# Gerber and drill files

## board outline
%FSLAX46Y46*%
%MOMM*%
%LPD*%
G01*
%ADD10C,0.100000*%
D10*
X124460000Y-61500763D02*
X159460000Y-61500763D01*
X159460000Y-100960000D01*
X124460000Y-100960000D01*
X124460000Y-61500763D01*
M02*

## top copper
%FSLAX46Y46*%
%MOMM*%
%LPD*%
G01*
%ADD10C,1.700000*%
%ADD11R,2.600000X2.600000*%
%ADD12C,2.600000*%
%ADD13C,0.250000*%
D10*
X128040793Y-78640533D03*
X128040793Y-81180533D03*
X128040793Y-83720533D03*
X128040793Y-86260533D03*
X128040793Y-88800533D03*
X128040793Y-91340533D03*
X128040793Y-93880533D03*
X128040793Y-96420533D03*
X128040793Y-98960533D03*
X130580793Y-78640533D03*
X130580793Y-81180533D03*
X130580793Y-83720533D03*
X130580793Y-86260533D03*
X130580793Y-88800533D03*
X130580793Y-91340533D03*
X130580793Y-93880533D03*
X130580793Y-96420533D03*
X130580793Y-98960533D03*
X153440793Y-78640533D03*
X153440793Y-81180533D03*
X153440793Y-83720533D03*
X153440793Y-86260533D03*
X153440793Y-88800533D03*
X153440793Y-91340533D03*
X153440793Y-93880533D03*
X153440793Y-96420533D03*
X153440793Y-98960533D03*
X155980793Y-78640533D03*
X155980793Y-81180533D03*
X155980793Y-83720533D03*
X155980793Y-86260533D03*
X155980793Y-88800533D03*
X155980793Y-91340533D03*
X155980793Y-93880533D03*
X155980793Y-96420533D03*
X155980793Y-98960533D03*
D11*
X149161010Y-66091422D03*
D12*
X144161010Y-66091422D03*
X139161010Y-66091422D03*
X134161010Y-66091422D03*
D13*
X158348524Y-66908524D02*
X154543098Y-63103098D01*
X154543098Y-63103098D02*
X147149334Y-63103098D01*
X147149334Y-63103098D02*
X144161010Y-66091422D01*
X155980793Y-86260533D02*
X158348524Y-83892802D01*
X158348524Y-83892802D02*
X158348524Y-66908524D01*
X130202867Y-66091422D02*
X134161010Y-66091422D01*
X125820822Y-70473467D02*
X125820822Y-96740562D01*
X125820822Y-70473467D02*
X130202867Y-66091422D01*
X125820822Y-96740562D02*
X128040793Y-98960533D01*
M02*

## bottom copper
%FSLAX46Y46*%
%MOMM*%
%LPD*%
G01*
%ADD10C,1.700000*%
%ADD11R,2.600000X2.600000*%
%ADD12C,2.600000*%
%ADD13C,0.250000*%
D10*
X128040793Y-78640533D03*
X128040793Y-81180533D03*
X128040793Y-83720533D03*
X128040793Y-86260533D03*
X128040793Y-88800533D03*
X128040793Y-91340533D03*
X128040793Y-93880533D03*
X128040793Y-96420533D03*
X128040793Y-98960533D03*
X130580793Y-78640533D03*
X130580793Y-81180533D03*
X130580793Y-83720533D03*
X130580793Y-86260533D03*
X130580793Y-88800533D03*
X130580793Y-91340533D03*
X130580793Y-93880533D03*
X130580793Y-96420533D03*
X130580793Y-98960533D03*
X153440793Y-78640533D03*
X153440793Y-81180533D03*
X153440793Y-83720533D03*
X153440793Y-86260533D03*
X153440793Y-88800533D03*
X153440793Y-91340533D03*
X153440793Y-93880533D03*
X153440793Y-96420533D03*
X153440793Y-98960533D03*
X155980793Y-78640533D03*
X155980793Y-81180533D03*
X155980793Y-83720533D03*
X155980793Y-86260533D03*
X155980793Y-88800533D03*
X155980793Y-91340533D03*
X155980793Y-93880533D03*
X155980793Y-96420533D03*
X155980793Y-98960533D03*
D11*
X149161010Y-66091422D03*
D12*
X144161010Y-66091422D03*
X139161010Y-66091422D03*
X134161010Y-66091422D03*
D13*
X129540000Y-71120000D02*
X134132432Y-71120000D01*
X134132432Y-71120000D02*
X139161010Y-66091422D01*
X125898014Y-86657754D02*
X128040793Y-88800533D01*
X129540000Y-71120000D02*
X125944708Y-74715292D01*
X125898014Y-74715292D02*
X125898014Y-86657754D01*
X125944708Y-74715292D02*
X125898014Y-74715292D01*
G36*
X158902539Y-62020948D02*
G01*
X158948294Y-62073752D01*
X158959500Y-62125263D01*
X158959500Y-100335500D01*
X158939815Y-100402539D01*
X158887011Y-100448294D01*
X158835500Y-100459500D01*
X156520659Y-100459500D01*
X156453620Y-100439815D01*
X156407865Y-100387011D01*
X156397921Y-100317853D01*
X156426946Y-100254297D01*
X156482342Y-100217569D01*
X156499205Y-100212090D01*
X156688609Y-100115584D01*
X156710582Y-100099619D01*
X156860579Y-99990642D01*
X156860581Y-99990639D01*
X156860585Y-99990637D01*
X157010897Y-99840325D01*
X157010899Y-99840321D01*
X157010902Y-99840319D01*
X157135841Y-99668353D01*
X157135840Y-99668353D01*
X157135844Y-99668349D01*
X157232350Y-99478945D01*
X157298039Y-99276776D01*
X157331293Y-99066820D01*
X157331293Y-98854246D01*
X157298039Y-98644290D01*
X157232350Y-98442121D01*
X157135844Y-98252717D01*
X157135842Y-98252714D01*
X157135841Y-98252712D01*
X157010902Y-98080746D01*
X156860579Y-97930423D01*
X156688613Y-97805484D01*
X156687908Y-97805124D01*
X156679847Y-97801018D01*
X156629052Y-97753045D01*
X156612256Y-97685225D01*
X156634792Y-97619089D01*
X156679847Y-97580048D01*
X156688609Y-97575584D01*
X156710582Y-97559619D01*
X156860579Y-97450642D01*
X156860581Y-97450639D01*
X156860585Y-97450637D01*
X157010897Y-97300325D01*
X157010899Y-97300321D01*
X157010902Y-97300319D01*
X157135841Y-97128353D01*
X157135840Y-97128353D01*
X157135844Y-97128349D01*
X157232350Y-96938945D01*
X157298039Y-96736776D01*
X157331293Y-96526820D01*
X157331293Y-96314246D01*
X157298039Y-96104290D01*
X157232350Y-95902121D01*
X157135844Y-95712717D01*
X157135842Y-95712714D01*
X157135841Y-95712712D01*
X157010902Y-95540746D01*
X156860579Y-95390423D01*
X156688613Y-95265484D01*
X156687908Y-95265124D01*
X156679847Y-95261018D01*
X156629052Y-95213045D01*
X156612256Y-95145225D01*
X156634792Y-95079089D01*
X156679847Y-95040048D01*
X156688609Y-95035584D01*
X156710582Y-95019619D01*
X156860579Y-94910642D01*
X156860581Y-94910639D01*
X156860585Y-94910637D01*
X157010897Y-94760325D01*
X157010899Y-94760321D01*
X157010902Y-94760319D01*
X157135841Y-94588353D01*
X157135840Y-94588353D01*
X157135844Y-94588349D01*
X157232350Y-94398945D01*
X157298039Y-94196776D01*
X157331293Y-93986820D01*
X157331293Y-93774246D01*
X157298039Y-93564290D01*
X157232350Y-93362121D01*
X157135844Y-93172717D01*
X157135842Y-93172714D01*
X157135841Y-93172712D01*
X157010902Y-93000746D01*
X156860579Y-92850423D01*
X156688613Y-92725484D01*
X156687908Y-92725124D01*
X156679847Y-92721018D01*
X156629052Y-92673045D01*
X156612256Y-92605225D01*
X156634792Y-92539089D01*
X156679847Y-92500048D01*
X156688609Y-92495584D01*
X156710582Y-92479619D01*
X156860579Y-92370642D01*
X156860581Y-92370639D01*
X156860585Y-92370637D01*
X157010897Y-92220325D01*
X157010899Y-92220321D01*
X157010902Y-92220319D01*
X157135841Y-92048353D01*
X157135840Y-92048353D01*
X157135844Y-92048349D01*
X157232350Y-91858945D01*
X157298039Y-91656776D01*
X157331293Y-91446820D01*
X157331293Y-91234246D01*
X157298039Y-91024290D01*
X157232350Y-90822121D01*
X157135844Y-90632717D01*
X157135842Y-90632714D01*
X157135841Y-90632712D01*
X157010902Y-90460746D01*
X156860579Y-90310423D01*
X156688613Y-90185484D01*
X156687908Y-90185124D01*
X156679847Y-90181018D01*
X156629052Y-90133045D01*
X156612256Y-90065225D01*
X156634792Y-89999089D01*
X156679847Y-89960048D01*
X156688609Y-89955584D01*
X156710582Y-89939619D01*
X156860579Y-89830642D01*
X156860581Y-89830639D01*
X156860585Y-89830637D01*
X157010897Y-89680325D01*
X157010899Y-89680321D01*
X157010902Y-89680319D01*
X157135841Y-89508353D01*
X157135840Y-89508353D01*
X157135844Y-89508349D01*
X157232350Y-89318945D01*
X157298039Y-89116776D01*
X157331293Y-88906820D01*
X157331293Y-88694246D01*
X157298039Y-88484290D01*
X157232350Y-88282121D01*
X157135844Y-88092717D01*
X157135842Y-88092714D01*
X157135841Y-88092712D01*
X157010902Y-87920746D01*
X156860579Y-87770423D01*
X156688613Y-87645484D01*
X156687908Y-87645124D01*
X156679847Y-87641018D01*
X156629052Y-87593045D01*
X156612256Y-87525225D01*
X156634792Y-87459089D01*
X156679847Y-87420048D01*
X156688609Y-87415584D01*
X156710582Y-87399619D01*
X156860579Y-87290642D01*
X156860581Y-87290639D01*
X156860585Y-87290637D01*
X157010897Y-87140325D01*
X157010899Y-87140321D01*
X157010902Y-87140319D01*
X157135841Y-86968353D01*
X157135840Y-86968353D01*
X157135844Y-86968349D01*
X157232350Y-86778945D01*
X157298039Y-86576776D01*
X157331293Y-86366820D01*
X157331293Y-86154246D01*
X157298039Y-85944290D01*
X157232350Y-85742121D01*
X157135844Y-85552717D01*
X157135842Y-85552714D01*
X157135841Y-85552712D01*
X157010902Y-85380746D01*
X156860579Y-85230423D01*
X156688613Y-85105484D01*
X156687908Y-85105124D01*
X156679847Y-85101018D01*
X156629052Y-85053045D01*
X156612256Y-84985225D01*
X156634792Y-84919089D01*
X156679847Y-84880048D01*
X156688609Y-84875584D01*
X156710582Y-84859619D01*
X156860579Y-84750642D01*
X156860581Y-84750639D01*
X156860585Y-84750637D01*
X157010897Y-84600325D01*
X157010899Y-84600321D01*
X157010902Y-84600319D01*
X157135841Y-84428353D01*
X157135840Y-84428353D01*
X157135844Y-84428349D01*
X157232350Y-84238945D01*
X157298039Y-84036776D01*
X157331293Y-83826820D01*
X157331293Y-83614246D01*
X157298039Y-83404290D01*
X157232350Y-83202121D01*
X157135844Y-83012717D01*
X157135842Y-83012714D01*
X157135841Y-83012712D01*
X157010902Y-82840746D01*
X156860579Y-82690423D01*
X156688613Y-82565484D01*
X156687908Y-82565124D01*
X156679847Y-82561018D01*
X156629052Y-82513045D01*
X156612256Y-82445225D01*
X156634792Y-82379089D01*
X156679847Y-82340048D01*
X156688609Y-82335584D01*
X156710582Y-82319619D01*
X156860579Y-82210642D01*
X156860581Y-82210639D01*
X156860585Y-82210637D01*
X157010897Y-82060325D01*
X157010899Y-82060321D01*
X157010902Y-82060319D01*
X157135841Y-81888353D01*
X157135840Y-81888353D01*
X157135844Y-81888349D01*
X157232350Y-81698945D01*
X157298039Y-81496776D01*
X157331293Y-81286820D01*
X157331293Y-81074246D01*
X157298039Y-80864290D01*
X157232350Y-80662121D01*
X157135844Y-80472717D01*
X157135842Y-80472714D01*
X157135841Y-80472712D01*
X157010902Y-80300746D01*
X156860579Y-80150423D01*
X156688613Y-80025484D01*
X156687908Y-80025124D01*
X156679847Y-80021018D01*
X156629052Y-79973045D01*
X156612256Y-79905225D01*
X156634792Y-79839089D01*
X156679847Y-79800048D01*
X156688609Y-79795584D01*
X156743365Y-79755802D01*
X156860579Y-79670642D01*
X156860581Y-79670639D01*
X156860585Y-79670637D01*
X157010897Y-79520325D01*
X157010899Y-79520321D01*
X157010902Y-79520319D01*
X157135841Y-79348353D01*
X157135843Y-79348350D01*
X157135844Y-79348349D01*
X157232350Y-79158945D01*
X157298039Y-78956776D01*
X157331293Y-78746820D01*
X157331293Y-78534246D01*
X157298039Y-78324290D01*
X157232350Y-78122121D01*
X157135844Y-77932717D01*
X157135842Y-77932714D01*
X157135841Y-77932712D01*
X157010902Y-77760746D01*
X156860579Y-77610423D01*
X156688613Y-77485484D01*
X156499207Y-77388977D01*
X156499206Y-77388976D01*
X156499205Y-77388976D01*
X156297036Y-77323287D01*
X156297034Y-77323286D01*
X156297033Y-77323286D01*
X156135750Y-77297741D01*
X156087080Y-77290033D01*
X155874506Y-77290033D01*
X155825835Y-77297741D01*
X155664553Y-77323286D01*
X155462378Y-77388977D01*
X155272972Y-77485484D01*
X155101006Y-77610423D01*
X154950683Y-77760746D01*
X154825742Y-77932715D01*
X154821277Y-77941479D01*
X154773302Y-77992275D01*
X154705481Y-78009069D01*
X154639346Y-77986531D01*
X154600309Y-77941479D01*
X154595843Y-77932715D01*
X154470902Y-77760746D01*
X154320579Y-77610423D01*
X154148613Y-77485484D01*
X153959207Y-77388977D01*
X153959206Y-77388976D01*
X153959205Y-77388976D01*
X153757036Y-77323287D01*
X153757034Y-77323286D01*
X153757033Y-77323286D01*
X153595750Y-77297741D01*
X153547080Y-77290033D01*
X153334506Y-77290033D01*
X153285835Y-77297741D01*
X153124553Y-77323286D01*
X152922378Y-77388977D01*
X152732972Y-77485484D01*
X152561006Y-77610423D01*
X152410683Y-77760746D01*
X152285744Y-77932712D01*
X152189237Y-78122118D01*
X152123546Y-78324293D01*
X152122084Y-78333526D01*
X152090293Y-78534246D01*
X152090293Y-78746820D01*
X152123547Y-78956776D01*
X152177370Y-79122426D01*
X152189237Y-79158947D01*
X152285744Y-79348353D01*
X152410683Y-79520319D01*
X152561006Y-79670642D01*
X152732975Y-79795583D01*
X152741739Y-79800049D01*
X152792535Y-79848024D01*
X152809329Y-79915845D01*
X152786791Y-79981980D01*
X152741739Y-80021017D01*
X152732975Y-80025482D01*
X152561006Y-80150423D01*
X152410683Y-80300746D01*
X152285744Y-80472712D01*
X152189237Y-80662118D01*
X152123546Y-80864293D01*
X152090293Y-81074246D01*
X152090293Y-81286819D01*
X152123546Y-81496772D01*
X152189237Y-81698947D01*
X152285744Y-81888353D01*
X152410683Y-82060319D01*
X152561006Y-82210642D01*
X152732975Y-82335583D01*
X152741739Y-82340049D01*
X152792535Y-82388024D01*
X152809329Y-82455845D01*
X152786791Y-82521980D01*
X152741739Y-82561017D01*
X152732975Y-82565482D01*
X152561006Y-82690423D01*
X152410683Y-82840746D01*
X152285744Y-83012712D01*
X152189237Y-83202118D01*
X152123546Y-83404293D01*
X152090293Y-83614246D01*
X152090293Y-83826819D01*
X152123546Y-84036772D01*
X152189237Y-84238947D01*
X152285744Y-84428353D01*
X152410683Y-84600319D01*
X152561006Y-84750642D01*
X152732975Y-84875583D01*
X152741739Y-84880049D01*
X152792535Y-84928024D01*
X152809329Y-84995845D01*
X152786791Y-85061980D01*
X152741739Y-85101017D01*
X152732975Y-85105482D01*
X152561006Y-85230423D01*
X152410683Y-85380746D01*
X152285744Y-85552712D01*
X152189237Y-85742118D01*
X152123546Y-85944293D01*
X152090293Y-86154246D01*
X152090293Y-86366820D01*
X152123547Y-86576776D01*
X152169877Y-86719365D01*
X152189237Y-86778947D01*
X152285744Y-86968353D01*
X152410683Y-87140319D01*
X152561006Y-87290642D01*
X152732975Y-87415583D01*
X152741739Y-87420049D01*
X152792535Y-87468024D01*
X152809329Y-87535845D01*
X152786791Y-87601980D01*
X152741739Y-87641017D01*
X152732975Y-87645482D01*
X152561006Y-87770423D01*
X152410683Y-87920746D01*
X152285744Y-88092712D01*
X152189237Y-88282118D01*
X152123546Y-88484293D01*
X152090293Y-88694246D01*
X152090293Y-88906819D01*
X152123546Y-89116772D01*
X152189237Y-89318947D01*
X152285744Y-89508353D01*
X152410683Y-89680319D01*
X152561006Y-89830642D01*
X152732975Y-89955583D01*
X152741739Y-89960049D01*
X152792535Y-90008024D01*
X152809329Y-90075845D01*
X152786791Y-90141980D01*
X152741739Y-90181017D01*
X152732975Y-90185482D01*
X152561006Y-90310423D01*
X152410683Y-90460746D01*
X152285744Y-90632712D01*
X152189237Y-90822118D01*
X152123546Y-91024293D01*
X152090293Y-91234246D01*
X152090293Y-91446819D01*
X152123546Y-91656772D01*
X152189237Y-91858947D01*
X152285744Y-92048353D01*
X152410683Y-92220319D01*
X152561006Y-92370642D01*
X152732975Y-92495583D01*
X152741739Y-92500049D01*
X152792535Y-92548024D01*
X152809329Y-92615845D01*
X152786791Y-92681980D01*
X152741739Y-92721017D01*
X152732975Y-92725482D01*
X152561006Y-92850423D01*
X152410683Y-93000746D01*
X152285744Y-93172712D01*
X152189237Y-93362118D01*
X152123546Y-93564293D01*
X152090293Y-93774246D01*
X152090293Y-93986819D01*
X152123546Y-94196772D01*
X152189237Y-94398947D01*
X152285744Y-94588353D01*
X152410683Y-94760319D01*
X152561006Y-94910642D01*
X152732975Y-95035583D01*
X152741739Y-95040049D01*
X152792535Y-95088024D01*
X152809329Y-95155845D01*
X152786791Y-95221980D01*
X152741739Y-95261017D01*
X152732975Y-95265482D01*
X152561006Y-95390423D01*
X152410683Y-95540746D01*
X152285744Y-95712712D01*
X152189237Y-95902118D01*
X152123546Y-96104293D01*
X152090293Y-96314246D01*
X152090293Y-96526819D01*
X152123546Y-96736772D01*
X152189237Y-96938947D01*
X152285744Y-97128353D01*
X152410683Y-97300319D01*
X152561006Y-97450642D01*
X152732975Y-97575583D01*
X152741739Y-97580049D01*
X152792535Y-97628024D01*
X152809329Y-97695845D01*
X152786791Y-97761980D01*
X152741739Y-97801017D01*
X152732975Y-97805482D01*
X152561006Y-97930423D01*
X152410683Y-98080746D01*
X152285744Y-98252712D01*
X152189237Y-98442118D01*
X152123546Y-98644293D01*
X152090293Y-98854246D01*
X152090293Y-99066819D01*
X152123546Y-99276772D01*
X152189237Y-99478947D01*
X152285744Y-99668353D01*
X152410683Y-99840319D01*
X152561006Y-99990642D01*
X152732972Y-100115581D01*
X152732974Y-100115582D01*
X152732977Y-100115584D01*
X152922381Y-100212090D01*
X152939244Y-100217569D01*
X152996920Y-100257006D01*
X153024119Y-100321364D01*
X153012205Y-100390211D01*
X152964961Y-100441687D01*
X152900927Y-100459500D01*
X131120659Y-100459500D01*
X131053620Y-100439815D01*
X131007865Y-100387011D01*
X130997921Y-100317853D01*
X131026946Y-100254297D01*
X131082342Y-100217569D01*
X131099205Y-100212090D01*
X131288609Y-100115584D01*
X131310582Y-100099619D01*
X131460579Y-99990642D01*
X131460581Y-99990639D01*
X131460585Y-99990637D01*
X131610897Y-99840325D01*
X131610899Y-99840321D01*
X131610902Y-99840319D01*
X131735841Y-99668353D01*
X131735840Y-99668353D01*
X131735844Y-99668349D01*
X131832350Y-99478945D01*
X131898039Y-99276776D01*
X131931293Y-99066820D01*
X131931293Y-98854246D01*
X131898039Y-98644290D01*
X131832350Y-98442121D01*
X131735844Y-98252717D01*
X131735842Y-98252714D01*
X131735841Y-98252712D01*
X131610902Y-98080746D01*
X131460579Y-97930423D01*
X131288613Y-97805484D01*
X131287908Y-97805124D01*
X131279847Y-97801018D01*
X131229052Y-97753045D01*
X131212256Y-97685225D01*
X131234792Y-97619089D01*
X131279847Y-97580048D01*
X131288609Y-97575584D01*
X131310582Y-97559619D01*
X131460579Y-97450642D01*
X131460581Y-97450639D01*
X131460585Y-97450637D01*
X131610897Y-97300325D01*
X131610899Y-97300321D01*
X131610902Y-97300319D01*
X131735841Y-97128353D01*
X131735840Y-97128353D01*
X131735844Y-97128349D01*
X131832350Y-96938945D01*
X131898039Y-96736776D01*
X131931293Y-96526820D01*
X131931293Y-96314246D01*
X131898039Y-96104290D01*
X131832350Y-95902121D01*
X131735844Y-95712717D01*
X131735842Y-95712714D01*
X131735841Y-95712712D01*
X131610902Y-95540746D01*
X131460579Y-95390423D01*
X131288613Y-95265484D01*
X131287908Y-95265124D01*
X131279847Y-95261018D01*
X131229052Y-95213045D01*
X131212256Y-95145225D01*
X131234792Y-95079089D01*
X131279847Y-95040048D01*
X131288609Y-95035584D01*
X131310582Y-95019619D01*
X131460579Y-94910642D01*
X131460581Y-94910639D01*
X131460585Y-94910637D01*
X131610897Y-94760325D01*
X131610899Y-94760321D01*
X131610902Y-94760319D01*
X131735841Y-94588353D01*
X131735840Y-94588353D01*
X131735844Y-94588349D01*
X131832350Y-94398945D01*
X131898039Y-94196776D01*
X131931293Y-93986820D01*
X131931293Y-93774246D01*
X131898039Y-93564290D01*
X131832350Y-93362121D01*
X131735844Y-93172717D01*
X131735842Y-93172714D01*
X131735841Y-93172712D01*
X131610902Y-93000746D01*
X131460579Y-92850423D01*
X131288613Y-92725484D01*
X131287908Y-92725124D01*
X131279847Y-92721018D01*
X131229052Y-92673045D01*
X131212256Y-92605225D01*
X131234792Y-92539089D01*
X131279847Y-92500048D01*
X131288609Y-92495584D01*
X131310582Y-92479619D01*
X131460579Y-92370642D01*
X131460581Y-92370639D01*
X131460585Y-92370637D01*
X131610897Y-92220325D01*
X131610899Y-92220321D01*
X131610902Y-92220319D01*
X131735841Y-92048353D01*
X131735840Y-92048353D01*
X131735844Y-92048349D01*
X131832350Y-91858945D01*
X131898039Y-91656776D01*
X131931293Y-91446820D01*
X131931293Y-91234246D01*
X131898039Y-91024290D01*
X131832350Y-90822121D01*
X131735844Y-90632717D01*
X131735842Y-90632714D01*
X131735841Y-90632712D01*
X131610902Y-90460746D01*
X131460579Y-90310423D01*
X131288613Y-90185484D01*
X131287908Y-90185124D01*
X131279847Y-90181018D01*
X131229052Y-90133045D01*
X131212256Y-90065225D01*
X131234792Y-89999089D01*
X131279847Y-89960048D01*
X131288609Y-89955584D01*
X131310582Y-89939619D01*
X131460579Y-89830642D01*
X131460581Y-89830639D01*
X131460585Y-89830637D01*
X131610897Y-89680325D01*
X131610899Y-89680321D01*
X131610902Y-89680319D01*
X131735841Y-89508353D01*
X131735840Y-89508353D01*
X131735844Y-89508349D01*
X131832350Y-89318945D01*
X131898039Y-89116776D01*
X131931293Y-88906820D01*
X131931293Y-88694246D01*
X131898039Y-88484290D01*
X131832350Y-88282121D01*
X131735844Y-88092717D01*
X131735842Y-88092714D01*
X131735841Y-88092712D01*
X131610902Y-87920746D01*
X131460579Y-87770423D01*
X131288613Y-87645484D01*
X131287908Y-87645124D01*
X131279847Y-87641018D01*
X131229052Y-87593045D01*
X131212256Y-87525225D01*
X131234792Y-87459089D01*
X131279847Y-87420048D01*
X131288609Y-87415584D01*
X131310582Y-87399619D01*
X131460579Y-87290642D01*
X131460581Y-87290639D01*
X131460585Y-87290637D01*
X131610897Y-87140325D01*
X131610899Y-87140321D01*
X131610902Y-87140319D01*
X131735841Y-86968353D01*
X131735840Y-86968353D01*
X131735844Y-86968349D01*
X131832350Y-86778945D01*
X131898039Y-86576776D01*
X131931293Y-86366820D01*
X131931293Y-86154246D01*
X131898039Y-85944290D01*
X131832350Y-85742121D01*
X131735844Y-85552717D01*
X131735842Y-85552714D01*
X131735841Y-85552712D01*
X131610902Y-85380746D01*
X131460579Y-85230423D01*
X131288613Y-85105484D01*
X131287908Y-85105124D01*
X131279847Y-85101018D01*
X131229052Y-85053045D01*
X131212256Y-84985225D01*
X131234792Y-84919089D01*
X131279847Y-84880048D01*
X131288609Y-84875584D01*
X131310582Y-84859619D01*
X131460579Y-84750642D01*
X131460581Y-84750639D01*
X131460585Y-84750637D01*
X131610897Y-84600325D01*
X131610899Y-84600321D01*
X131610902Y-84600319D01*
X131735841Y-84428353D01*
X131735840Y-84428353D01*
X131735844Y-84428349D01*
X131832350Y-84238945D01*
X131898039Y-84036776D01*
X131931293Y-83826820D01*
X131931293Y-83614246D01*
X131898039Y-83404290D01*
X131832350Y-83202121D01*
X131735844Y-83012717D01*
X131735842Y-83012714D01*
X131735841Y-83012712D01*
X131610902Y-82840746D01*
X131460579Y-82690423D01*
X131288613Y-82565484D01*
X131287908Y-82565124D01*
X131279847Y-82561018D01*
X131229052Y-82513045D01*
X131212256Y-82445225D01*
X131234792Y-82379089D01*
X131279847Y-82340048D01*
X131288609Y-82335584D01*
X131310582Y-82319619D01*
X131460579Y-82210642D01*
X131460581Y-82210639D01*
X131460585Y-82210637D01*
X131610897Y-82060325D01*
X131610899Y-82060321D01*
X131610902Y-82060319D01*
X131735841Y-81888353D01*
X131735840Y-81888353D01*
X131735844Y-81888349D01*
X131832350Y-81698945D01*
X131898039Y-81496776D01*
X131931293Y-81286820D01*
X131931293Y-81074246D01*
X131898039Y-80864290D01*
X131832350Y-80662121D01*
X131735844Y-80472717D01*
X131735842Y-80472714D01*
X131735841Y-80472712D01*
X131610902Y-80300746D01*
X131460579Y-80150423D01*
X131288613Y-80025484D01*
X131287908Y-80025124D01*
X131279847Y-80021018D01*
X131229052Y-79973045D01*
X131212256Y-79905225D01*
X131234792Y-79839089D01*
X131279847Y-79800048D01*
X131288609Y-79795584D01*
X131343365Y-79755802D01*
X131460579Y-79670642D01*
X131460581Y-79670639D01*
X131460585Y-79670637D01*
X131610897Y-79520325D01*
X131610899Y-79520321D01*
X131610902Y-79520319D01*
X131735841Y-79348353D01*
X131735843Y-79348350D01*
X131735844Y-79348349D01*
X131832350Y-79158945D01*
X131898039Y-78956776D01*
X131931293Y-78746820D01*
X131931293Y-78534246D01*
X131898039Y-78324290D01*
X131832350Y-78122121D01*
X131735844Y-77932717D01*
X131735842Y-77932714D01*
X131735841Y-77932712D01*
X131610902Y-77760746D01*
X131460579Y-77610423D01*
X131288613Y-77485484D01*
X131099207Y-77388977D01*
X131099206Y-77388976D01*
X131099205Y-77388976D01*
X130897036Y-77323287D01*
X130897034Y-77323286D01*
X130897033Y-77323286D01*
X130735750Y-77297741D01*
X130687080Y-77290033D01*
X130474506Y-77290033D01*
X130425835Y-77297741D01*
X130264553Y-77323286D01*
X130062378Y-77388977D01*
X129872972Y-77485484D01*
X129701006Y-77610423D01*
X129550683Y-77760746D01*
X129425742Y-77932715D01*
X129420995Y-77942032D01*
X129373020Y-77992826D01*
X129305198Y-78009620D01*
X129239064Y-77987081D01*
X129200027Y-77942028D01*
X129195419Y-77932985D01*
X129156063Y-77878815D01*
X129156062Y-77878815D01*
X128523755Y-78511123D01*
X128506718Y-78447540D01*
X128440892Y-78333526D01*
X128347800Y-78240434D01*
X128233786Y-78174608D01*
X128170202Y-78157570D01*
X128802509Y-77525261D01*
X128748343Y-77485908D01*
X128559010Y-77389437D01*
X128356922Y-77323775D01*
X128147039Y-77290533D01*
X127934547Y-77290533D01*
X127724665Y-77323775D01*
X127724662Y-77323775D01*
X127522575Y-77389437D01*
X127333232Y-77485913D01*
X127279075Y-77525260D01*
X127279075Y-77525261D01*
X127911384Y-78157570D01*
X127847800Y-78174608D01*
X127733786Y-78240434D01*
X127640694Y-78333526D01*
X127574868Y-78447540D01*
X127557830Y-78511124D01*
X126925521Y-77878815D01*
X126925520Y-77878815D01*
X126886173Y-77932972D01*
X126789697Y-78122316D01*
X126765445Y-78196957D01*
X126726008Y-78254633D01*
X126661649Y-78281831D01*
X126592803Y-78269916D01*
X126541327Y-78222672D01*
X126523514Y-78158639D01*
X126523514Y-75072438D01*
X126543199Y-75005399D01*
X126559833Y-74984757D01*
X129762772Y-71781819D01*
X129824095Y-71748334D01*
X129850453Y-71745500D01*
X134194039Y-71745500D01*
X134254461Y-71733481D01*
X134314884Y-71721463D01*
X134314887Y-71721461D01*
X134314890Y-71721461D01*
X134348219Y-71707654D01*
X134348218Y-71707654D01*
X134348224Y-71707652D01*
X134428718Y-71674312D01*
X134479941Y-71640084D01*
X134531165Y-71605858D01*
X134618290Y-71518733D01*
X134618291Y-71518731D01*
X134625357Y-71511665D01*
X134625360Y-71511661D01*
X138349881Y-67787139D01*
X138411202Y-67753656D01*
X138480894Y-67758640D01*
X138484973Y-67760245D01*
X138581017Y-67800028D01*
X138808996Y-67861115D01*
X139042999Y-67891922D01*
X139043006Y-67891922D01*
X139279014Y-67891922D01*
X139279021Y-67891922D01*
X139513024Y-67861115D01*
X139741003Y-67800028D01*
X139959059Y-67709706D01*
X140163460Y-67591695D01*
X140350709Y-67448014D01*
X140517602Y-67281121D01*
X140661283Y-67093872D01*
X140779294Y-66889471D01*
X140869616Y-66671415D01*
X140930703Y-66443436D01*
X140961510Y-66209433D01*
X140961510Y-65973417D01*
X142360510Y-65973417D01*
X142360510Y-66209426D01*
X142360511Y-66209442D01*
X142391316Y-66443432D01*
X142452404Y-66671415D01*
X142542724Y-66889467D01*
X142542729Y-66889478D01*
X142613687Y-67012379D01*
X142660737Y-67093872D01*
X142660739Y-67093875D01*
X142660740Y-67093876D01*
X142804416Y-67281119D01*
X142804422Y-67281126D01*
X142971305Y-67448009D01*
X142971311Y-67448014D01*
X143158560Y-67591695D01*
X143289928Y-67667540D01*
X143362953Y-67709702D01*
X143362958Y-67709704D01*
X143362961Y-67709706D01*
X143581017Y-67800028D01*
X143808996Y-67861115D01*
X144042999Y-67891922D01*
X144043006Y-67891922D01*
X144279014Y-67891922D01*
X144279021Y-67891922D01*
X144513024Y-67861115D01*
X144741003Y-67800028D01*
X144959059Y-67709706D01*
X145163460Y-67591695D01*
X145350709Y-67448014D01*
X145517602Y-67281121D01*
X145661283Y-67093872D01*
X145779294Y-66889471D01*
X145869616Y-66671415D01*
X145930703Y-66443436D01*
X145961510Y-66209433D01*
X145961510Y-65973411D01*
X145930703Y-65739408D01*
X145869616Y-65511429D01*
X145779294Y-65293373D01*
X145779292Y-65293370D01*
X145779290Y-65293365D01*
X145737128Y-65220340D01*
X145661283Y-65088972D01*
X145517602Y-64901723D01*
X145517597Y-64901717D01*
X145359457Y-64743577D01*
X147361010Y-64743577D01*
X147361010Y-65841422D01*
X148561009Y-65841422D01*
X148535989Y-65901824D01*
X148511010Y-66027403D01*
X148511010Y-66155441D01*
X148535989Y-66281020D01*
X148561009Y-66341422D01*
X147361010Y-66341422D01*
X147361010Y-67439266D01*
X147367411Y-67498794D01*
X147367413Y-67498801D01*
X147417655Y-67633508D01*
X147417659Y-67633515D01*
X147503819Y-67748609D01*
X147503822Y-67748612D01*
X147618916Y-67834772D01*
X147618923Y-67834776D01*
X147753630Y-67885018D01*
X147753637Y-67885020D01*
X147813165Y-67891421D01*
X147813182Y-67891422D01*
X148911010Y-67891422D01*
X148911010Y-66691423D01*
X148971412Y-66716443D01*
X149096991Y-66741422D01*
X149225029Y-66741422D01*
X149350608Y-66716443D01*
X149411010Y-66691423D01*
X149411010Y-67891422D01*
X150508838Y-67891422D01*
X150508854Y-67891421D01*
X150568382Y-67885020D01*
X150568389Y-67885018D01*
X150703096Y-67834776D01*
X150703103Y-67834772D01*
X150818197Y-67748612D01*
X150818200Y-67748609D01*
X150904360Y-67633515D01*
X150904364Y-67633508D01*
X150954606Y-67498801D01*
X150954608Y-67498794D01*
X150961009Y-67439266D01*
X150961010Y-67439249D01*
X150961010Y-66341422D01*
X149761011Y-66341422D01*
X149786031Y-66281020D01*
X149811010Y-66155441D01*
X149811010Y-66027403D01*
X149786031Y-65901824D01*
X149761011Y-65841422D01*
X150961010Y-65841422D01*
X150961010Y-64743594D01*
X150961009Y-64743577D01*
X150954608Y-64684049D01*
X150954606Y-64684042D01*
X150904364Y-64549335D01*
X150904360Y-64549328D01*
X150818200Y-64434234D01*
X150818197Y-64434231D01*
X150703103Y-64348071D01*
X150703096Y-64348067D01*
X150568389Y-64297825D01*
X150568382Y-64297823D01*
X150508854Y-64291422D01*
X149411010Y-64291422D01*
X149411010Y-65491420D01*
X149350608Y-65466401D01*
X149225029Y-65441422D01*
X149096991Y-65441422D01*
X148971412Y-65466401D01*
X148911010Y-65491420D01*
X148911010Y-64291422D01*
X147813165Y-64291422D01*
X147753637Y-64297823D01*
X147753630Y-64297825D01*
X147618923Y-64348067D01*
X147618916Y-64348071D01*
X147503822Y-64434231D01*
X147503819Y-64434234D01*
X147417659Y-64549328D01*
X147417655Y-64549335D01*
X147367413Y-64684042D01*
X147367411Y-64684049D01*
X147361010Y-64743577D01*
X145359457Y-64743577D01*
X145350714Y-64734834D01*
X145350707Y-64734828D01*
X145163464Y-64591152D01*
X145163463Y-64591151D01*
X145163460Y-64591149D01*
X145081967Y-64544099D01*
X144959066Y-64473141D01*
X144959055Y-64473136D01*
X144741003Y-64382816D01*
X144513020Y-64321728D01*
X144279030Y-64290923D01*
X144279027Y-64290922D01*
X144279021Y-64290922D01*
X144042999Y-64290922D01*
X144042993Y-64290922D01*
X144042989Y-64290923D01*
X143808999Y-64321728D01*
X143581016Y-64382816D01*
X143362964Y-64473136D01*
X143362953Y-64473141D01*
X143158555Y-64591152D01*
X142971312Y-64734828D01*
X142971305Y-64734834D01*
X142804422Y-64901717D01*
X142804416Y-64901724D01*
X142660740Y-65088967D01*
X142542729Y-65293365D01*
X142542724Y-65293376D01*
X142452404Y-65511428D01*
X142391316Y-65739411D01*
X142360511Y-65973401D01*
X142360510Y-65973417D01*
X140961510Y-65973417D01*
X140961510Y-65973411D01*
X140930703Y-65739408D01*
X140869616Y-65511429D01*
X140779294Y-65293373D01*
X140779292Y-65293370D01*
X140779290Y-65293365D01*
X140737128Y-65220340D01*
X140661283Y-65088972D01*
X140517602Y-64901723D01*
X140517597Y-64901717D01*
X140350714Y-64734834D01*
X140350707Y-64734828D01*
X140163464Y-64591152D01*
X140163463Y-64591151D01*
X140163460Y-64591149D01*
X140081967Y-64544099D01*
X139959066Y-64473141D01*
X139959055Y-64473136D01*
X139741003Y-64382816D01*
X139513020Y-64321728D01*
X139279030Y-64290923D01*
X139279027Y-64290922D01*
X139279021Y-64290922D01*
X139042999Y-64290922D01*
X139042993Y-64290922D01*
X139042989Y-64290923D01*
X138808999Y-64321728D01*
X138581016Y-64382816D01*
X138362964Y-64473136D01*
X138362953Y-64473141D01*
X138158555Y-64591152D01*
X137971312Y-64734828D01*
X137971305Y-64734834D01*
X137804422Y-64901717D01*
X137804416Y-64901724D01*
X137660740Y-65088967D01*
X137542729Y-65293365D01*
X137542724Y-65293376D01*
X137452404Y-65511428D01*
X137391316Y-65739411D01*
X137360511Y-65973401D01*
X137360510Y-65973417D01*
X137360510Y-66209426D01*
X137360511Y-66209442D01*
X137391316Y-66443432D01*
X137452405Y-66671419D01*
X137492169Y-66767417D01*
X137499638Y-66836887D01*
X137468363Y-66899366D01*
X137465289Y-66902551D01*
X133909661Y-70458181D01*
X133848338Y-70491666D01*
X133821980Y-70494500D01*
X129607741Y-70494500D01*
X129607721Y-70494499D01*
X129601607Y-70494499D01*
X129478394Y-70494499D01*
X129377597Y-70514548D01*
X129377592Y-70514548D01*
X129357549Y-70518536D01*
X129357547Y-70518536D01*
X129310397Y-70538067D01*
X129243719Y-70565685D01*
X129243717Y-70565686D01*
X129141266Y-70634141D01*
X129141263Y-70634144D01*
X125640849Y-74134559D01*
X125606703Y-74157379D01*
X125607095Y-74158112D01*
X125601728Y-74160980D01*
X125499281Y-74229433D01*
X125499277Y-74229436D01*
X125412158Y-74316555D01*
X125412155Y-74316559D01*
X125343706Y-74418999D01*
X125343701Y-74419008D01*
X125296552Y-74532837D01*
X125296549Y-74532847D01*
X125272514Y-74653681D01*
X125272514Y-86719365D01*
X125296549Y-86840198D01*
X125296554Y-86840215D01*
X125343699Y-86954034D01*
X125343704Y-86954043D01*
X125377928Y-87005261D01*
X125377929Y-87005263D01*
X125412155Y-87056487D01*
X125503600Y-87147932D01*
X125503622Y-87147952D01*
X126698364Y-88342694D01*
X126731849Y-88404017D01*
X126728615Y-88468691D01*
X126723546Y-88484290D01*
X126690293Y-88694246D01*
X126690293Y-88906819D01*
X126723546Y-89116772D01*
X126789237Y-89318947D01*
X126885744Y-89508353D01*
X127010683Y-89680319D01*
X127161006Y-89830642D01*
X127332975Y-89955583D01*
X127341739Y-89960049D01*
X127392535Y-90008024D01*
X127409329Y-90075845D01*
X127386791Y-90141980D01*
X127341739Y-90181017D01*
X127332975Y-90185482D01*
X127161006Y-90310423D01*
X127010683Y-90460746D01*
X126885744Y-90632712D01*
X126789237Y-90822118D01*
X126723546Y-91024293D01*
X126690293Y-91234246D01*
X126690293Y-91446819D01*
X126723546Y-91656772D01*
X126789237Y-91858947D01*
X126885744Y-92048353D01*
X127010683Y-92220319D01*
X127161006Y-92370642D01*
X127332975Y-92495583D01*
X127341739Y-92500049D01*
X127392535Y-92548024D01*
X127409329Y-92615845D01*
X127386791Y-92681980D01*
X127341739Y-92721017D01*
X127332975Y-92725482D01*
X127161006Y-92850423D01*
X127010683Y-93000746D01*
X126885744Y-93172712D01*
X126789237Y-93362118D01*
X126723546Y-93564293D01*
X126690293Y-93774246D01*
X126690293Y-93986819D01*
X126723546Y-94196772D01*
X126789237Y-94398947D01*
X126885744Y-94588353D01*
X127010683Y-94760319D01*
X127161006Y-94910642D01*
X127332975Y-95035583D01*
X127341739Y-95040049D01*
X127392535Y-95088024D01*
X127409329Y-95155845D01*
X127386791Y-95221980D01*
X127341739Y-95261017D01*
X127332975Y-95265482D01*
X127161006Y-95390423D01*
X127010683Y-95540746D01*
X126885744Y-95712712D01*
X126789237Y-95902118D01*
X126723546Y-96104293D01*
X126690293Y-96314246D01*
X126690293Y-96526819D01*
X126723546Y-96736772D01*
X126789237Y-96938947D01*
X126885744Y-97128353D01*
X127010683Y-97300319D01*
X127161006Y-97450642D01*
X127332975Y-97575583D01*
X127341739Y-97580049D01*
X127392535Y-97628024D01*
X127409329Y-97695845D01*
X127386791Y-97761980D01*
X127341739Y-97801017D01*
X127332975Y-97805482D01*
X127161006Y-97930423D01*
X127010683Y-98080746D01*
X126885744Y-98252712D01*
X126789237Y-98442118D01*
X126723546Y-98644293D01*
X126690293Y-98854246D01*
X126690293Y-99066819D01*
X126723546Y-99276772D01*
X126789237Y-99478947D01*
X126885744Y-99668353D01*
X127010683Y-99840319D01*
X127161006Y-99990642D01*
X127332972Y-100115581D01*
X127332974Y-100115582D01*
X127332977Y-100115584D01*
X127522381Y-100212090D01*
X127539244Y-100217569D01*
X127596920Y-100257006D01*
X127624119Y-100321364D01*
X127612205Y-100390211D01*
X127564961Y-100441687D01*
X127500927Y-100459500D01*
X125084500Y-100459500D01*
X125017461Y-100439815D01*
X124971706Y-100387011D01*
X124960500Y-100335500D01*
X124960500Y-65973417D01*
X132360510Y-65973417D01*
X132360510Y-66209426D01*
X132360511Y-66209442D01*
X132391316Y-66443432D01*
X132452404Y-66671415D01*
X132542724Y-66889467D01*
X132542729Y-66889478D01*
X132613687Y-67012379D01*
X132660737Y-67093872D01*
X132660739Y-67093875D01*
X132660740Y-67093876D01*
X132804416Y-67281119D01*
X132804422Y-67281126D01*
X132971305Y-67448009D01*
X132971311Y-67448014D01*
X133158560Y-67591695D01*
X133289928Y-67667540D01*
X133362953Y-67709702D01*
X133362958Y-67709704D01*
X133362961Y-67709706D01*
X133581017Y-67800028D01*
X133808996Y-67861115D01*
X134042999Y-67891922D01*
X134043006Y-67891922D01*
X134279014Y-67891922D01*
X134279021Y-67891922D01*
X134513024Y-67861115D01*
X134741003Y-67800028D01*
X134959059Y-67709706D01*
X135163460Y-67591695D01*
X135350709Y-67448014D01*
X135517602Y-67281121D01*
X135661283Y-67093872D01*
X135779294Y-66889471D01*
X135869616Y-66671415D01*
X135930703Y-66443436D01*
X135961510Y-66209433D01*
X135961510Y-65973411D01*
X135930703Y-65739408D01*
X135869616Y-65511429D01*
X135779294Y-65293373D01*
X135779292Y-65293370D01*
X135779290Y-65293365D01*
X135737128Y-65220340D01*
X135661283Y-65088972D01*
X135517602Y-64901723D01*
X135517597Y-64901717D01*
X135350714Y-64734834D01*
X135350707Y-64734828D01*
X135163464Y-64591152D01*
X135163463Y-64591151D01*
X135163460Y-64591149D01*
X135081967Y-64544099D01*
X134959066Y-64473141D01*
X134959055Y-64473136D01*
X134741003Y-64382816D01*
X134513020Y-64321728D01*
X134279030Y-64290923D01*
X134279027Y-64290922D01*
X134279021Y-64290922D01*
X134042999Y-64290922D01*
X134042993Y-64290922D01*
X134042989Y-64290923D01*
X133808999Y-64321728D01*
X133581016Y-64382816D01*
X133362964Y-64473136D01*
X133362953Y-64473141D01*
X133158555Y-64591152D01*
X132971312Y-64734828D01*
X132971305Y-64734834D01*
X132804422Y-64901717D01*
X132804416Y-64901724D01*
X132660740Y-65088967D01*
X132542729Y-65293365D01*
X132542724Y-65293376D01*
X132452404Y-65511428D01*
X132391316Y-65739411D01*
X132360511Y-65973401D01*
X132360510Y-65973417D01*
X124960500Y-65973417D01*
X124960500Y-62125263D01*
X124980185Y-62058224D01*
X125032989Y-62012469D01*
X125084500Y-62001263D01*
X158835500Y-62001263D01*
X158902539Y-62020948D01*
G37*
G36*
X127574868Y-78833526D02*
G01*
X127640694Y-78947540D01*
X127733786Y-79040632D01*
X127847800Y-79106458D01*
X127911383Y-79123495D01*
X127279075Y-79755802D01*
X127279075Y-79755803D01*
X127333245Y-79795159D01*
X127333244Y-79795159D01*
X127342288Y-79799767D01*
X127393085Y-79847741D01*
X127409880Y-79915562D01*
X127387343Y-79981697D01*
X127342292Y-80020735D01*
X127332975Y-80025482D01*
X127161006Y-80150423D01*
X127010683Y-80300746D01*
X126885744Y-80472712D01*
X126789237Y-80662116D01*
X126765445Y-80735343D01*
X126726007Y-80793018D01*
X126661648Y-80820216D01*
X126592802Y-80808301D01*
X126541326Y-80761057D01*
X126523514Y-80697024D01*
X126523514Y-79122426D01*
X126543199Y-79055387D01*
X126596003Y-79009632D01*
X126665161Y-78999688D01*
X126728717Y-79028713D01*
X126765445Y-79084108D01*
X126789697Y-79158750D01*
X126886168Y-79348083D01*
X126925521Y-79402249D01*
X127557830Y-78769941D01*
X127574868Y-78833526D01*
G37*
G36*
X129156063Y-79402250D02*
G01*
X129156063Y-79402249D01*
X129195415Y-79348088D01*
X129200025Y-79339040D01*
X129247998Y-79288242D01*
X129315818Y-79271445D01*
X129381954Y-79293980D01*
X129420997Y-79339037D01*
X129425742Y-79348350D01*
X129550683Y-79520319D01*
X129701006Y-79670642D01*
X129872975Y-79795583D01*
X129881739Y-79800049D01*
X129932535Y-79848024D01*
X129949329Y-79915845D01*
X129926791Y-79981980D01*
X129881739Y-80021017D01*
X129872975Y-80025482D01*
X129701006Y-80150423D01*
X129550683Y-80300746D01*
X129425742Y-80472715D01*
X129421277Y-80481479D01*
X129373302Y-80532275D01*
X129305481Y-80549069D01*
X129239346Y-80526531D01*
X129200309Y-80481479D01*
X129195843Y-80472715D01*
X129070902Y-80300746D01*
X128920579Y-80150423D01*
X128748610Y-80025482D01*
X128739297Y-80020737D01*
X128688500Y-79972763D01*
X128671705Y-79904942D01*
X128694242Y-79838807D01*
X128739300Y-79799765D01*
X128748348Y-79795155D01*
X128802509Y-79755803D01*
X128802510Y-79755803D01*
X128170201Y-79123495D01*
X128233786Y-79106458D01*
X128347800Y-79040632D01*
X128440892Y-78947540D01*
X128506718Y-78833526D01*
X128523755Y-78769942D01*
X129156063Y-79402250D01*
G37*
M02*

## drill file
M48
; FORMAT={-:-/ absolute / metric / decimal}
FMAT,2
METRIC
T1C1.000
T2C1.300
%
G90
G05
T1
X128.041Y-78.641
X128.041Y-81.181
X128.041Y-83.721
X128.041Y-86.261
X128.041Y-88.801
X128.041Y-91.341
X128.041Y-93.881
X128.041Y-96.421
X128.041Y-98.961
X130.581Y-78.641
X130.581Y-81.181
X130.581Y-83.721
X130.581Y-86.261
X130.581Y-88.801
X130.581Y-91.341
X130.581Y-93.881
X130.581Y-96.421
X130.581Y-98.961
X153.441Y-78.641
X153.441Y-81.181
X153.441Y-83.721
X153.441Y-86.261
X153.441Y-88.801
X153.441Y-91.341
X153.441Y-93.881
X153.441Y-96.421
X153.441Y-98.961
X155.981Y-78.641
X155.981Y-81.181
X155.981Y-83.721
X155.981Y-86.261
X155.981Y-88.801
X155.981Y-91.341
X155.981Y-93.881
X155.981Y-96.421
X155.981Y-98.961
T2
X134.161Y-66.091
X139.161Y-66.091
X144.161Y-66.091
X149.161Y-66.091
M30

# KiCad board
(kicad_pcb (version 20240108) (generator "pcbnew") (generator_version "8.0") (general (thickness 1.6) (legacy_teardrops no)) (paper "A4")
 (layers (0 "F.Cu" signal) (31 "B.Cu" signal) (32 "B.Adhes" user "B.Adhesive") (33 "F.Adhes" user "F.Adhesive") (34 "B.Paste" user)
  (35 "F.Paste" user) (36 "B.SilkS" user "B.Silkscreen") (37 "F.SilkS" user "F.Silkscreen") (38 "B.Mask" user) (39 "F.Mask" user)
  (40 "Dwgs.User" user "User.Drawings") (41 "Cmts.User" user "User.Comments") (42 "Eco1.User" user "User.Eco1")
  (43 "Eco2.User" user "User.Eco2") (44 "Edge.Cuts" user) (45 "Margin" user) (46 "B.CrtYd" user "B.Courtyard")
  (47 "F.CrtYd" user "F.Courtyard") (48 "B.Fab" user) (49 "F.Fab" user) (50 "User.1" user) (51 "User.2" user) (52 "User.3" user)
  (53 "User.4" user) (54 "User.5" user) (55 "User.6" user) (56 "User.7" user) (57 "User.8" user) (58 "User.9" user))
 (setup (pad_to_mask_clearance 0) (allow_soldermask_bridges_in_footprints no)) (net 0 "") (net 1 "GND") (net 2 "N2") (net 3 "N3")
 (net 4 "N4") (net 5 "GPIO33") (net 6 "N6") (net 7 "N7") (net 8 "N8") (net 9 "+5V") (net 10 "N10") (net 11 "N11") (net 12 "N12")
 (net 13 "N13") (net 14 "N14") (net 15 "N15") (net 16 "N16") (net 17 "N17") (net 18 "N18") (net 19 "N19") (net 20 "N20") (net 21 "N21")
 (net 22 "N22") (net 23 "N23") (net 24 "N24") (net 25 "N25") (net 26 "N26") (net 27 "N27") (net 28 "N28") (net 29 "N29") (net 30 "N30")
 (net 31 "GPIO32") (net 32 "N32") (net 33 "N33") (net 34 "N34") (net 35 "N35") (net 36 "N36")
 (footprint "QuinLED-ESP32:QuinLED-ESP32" (layer "F.Cu") (at 142.112393 93.220133)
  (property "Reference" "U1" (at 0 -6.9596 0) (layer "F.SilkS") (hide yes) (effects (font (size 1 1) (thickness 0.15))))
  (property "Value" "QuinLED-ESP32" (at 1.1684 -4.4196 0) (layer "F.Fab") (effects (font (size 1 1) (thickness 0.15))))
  (pad "1" thru_hole circle (at -14.0716 -14.5796) (size 1.7 1.7) (drill 1) (layers "*.Cu" "*.Mask") (remove_unused_layers no) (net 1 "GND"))
  (pad "2" thru_hole circle (at -14.0716 -12.0396) (size 1.7 1.7) (drill 1) (layers "*.Cu" "*.Mask") (remove_unused_layers no) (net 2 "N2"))
  (pad "3" thru_hole circle (at -14.0716 -9.4996) (size 1.7 1.7) (drill 1) (layers "*.Cu" "*.Mask") (remove_unused_layers no) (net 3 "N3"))
  (pad "4" thru_hole circle (at -14.0716 -6.9596) (size 1.7 1.7) (drill 1) (layers "*.Cu" "*.Mask") (remove_unused_layers no) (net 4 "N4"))
  (pad "5" thru_hole circle (at -14.0716 -4.4196) (size 1.7 1.7) (drill 1) (layers "*.Cu" "*.Mask") (remove_unused_layers no)
   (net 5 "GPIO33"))
  (pad "6" thru_hole circle (at -14.0716 -1.8796) (size 1.7 1.7) (drill 1) (layers "*.Cu" "*.Mask") (remove_unused_layers no) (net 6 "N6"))
  (pad "7" thru_hole circle (at -14.0716 0.6604) (size 1.7 1.7) (drill 1) (layers "*.Cu" "*.Mask") (remove_unused_layers no) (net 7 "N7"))
  (pad "8" thru_hole circle (at -14.0716 3.2004) (size 1.7 1.7) (drill 1) (layers "*.Cu" "*.Mask") (remove_unused_layers no) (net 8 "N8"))
  (pad "9" thru_hole circle (at -14.0716 5.7404) (size 1.7 1.7) (drill 1) (layers "*.Cu" "*.Mask") (remove_unused_layers no) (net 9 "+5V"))
  (pad "10" thru_hole circle (at -11.5316 -14.5796) (size 1.7 1.7) (drill 1) (layers "*.Cu" "*.Mask") (remove_unused_layers no)
   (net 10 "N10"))
  (pad "11" thru_hole circle (at -11.5316 -12.0396) (size 1.7 1.7) (drill 1) (layers "*.Cu" "*.Mask") (remove_unused_layers no)
   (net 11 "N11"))
  (pad "12" thru_hole circle (at -11.5316 -9.4996) (size 1.7 1.7) (drill 1) (layers "*.Cu" "*.Mask") (remove_unused_layers no)
   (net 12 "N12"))
  (pad "13" thru_hole circle (at -11.5316 -6.9596) (size 1.7 1.7) (drill 1) (layers "*.Cu" "*.Mask") (remove_unused_layers no)
   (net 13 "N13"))
  (pad "14" thru_hole circle (at -11.5316 -4.4196) (size 1.7 1.7) (drill 1) (layers "*.Cu" "*.Mask") (remove_unused_layers no)
   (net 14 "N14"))
  (pad "15" thru_hole circle (at -11.5316 -1.8796) (size 1.7 1.7) (drill 1) (layers "*.Cu" "*.Mask") (remove_unused_layers no)
   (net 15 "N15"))
  (pad "16" thru_hole circle (at -11.5316 0.6604) (size 1.7 1.7) (drill 1) (layers "*.Cu" "*.Mask") (remove_unused_layers no) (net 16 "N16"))
  (pad "17" thru_hole circle (at -11.5316 3.2004) (size 1.7 1.7) (drill 1) (layers "*.Cu" "*.Mask") (remove_unused_layers no) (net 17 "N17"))
  (pad "18" thru_hole circle (at -11.5316 5.7404) (size 1.7 1.7) (drill 1) (layers "*.Cu" "*.Mask") (remove_unused_layers no) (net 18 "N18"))
  (pad "19" thru_hole circle (at 11.3284 -14.5796) (size 1.7 1.7) (drill 1) (layers "*.Cu" "*.Mask") (remove_unused_layers no)
   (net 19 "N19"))
  (pad "20" thru_hole circle (at 11.3284 -12.0396) (size 1.7 1.7) (drill 1) (layers "*.Cu" "*.Mask") (remove_unused_layers no)
   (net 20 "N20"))
  (pad "21" thru_hole circle (at 11.3284 -9.4996) (size 1.7 1.7) (drill 1) (layers "*.Cu" "*.Mask") (remove_unused_layers no) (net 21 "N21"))
  (pad "22" thru_hole circle (at 11.3284 -6.9596) (size 1.7 1.7) (drill 1) (layers "*.Cu" "*.Mask") (remove_unused_layers no) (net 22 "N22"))
  (pad "23" thru_hole circle (at 11.3284 -4.4196) (size 1.7 1.7) (drill 1) (layers "*.Cu" "*.Mask") (remove_unused_layers no) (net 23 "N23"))
  (pad "24" thru_hole circle (at 11.3284 -1.8796) (size 1.7 1.7) (drill 1) (layers "*.Cu" "*.Mask") (remove_unused_layers no) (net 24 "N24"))
  (pad "25" thru_hole circle (at 11.3284 0.6604) (size 1.7 1.7) (drill 1) (layers "*.Cu" "*.Mask") (remove_unused_layers no) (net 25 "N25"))
  (pad "26" thru_hole circle (at 11.3284 3.2004) (size 1.7 1.7) (drill 1) (layers "*.Cu" "*.Mask") (remove_unused_layers no) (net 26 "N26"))
  (pad "27" thru_hole circle (at 11.3284 5.7404) (size 1.7 1.7) (drill 1) (layers "*.Cu" "*.Mask") (remove_unused_layers no) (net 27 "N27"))
  (pad "28" thru_hole circle (at 13.8684 -14.5796) (size 1.7 1.7) (drill 1) (layers "*.Cu" "*.Mask") (remove_unused_layers no)
   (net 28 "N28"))
  (pad "29" thru_hole circle (at 13.8684 -12.0396) (size 1.7 1.7) (drill 1) (layers "*.Cu" "*.Mask") (remove_unused_layers no)
   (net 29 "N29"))
  (pad "30" thru_hole circle (at 13.8684 -9.4996) (size 1.7 1.7) (drill 1) (layers "*.Cu" "*.Mask") (remove_unused_layers no) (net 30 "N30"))
  (pad "31" thru_hole circle (at 13.8684 -6.9596) (size 1.7 1.7) (drill 1) (layers "*.Cu" "*.Mask") (remove_unused_layers no)
   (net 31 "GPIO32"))
  (pad "32" thru_hole circle (at 13.8684 -4.4196) (size 1.7 1.7) (drill 1) (layers "*.Cu" "*.Mask") (remove_unused_layers no) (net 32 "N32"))
  (pad "33" thru_hole circle (at 13.8684 -1.8796) (size 1.7 1.7) (drill 1) (layers "*.Cu" "*.Mask") (remove_unused_layers no) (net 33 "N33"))
  (pad "34" thru_hole circle (at 13.8684 0.6604) (size 1.7 1.7) (drill 1) (layers "*.Cu" "*.Mask") (remove_unused_layers no) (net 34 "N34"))
  (pad "35" thru_hole circle (at 13.8684 3.2004) (size 1.7 1.7) (drill 1) (layers "*.Cu" "*.Mask") (remove_unused_layers no) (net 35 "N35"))
  (pad "36" thru_hole circle (at 13.8684 5.7404) (size 1.7 1.7) (drill 1) (layers "*.Cu" "*.Mask") (remove_unused_layers no) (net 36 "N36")))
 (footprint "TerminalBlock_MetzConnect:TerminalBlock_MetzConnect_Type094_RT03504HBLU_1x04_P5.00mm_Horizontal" (layer "F.Cu")
  (at 149.16101 66.091422 180)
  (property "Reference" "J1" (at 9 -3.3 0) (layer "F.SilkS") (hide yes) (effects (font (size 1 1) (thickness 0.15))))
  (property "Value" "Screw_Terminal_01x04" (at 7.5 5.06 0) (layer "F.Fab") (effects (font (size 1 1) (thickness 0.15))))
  (pad "1" thru_hole rect (at 0 0 180) (size 2.6 2.6) (drill 1.3) (layers "*.Cu" "*.Mask") (remove_unused_layers no) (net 1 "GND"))
  (pad "2" thru_hole circle (at 5 0 180) (size 2.6 2.6) (drill 1.3) (layers "*.Cu" "*.Mask") (remove_unused_layers no) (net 31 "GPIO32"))
  (pad "3" thru_hole circle (at 10 0 180) (size 2.6 2.6) (drill 1.3) (layers "*.Cu" "*.Mask") (remove_unused_layers no) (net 5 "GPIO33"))
  (pad "4" thru_hole circle (at 15 0 180) (size 2.6 2.6) (drill 1.3) (layers "*.Cu" "*.Mask") (remove_unused_layers no) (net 9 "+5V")))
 (gr_rect (start 124.46 61.500763) (end 159.46 100.96) (stroke (width 0.1) (type default)) (fill none) (layer "Edge.Cuts"))
 (segment (start 129.54 71.12) (end 134.132432 71.12) (width 0.25) (layer "B.Cu") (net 5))
 (segment (start 134.132432 71.12) (end 139.16101 66.091422) (width 0.25) (layer "B.Cu") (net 5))
 (segment (start 125.898014 86.657754) (end 128.040793 88.800533) (width 0.25) (layer "B.Cu") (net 5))
 (segment (start 129.54 71.12) (end 125.944708 74.715292) (width 0.25) (layer "B.Cu") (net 5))
 (segment (start 125.898014 74.715292) (end 125.898014 86.657754) (width 0.25) (layer "B.Cu") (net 5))
 (segment (start 125.944708 74.715292) (end 125.898014 74.715292) (width 0.25) (layer "B.Cu") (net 5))
 (segment (start 158.348524 66.908524) (end 154.543098 63.103098) (width 0.25) (layer "F.Cu") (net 31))
 (segment (start 154.543098 63.103098) (end 147.149334 63.103098) (width 0.25) (layer "F.Cu") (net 31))
 (segment (start 147.149334 63.103098) (end 144.16101 66.091422) (width 0.25) (layer "F.Cu") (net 31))
 (segment (start 155.980793 86.260533) (end 158.348524 83.892802) (width 0.25) (layer "F.Cu") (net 31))
 (segment (start 158.348524 83.892802) (end 158.348524 66.908524) (width 0.25) (layer "F.Cu") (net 31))
 (segment (start 130.202867 66.091422) (end 134.16101 66.091422) (width 0.25) (layer "F.Cu") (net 9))
 (segment (start 125.820822 70.473467) (end 125.820822 96.740562) (width 0.25) (layer "F.Cu") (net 9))
 (segment (start 125.820822 70.473467) (end 130.202867 66.091422) (width 0.25) (layer "F.Cu") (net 9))
 (segment (start 125.820822 96.740562) (end 128.040793 98.960533) (width 0.25) (layer "F.Cu") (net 9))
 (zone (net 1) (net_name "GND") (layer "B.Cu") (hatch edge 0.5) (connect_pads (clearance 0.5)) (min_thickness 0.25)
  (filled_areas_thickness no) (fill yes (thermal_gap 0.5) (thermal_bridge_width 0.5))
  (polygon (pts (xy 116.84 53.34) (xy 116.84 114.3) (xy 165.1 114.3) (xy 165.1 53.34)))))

